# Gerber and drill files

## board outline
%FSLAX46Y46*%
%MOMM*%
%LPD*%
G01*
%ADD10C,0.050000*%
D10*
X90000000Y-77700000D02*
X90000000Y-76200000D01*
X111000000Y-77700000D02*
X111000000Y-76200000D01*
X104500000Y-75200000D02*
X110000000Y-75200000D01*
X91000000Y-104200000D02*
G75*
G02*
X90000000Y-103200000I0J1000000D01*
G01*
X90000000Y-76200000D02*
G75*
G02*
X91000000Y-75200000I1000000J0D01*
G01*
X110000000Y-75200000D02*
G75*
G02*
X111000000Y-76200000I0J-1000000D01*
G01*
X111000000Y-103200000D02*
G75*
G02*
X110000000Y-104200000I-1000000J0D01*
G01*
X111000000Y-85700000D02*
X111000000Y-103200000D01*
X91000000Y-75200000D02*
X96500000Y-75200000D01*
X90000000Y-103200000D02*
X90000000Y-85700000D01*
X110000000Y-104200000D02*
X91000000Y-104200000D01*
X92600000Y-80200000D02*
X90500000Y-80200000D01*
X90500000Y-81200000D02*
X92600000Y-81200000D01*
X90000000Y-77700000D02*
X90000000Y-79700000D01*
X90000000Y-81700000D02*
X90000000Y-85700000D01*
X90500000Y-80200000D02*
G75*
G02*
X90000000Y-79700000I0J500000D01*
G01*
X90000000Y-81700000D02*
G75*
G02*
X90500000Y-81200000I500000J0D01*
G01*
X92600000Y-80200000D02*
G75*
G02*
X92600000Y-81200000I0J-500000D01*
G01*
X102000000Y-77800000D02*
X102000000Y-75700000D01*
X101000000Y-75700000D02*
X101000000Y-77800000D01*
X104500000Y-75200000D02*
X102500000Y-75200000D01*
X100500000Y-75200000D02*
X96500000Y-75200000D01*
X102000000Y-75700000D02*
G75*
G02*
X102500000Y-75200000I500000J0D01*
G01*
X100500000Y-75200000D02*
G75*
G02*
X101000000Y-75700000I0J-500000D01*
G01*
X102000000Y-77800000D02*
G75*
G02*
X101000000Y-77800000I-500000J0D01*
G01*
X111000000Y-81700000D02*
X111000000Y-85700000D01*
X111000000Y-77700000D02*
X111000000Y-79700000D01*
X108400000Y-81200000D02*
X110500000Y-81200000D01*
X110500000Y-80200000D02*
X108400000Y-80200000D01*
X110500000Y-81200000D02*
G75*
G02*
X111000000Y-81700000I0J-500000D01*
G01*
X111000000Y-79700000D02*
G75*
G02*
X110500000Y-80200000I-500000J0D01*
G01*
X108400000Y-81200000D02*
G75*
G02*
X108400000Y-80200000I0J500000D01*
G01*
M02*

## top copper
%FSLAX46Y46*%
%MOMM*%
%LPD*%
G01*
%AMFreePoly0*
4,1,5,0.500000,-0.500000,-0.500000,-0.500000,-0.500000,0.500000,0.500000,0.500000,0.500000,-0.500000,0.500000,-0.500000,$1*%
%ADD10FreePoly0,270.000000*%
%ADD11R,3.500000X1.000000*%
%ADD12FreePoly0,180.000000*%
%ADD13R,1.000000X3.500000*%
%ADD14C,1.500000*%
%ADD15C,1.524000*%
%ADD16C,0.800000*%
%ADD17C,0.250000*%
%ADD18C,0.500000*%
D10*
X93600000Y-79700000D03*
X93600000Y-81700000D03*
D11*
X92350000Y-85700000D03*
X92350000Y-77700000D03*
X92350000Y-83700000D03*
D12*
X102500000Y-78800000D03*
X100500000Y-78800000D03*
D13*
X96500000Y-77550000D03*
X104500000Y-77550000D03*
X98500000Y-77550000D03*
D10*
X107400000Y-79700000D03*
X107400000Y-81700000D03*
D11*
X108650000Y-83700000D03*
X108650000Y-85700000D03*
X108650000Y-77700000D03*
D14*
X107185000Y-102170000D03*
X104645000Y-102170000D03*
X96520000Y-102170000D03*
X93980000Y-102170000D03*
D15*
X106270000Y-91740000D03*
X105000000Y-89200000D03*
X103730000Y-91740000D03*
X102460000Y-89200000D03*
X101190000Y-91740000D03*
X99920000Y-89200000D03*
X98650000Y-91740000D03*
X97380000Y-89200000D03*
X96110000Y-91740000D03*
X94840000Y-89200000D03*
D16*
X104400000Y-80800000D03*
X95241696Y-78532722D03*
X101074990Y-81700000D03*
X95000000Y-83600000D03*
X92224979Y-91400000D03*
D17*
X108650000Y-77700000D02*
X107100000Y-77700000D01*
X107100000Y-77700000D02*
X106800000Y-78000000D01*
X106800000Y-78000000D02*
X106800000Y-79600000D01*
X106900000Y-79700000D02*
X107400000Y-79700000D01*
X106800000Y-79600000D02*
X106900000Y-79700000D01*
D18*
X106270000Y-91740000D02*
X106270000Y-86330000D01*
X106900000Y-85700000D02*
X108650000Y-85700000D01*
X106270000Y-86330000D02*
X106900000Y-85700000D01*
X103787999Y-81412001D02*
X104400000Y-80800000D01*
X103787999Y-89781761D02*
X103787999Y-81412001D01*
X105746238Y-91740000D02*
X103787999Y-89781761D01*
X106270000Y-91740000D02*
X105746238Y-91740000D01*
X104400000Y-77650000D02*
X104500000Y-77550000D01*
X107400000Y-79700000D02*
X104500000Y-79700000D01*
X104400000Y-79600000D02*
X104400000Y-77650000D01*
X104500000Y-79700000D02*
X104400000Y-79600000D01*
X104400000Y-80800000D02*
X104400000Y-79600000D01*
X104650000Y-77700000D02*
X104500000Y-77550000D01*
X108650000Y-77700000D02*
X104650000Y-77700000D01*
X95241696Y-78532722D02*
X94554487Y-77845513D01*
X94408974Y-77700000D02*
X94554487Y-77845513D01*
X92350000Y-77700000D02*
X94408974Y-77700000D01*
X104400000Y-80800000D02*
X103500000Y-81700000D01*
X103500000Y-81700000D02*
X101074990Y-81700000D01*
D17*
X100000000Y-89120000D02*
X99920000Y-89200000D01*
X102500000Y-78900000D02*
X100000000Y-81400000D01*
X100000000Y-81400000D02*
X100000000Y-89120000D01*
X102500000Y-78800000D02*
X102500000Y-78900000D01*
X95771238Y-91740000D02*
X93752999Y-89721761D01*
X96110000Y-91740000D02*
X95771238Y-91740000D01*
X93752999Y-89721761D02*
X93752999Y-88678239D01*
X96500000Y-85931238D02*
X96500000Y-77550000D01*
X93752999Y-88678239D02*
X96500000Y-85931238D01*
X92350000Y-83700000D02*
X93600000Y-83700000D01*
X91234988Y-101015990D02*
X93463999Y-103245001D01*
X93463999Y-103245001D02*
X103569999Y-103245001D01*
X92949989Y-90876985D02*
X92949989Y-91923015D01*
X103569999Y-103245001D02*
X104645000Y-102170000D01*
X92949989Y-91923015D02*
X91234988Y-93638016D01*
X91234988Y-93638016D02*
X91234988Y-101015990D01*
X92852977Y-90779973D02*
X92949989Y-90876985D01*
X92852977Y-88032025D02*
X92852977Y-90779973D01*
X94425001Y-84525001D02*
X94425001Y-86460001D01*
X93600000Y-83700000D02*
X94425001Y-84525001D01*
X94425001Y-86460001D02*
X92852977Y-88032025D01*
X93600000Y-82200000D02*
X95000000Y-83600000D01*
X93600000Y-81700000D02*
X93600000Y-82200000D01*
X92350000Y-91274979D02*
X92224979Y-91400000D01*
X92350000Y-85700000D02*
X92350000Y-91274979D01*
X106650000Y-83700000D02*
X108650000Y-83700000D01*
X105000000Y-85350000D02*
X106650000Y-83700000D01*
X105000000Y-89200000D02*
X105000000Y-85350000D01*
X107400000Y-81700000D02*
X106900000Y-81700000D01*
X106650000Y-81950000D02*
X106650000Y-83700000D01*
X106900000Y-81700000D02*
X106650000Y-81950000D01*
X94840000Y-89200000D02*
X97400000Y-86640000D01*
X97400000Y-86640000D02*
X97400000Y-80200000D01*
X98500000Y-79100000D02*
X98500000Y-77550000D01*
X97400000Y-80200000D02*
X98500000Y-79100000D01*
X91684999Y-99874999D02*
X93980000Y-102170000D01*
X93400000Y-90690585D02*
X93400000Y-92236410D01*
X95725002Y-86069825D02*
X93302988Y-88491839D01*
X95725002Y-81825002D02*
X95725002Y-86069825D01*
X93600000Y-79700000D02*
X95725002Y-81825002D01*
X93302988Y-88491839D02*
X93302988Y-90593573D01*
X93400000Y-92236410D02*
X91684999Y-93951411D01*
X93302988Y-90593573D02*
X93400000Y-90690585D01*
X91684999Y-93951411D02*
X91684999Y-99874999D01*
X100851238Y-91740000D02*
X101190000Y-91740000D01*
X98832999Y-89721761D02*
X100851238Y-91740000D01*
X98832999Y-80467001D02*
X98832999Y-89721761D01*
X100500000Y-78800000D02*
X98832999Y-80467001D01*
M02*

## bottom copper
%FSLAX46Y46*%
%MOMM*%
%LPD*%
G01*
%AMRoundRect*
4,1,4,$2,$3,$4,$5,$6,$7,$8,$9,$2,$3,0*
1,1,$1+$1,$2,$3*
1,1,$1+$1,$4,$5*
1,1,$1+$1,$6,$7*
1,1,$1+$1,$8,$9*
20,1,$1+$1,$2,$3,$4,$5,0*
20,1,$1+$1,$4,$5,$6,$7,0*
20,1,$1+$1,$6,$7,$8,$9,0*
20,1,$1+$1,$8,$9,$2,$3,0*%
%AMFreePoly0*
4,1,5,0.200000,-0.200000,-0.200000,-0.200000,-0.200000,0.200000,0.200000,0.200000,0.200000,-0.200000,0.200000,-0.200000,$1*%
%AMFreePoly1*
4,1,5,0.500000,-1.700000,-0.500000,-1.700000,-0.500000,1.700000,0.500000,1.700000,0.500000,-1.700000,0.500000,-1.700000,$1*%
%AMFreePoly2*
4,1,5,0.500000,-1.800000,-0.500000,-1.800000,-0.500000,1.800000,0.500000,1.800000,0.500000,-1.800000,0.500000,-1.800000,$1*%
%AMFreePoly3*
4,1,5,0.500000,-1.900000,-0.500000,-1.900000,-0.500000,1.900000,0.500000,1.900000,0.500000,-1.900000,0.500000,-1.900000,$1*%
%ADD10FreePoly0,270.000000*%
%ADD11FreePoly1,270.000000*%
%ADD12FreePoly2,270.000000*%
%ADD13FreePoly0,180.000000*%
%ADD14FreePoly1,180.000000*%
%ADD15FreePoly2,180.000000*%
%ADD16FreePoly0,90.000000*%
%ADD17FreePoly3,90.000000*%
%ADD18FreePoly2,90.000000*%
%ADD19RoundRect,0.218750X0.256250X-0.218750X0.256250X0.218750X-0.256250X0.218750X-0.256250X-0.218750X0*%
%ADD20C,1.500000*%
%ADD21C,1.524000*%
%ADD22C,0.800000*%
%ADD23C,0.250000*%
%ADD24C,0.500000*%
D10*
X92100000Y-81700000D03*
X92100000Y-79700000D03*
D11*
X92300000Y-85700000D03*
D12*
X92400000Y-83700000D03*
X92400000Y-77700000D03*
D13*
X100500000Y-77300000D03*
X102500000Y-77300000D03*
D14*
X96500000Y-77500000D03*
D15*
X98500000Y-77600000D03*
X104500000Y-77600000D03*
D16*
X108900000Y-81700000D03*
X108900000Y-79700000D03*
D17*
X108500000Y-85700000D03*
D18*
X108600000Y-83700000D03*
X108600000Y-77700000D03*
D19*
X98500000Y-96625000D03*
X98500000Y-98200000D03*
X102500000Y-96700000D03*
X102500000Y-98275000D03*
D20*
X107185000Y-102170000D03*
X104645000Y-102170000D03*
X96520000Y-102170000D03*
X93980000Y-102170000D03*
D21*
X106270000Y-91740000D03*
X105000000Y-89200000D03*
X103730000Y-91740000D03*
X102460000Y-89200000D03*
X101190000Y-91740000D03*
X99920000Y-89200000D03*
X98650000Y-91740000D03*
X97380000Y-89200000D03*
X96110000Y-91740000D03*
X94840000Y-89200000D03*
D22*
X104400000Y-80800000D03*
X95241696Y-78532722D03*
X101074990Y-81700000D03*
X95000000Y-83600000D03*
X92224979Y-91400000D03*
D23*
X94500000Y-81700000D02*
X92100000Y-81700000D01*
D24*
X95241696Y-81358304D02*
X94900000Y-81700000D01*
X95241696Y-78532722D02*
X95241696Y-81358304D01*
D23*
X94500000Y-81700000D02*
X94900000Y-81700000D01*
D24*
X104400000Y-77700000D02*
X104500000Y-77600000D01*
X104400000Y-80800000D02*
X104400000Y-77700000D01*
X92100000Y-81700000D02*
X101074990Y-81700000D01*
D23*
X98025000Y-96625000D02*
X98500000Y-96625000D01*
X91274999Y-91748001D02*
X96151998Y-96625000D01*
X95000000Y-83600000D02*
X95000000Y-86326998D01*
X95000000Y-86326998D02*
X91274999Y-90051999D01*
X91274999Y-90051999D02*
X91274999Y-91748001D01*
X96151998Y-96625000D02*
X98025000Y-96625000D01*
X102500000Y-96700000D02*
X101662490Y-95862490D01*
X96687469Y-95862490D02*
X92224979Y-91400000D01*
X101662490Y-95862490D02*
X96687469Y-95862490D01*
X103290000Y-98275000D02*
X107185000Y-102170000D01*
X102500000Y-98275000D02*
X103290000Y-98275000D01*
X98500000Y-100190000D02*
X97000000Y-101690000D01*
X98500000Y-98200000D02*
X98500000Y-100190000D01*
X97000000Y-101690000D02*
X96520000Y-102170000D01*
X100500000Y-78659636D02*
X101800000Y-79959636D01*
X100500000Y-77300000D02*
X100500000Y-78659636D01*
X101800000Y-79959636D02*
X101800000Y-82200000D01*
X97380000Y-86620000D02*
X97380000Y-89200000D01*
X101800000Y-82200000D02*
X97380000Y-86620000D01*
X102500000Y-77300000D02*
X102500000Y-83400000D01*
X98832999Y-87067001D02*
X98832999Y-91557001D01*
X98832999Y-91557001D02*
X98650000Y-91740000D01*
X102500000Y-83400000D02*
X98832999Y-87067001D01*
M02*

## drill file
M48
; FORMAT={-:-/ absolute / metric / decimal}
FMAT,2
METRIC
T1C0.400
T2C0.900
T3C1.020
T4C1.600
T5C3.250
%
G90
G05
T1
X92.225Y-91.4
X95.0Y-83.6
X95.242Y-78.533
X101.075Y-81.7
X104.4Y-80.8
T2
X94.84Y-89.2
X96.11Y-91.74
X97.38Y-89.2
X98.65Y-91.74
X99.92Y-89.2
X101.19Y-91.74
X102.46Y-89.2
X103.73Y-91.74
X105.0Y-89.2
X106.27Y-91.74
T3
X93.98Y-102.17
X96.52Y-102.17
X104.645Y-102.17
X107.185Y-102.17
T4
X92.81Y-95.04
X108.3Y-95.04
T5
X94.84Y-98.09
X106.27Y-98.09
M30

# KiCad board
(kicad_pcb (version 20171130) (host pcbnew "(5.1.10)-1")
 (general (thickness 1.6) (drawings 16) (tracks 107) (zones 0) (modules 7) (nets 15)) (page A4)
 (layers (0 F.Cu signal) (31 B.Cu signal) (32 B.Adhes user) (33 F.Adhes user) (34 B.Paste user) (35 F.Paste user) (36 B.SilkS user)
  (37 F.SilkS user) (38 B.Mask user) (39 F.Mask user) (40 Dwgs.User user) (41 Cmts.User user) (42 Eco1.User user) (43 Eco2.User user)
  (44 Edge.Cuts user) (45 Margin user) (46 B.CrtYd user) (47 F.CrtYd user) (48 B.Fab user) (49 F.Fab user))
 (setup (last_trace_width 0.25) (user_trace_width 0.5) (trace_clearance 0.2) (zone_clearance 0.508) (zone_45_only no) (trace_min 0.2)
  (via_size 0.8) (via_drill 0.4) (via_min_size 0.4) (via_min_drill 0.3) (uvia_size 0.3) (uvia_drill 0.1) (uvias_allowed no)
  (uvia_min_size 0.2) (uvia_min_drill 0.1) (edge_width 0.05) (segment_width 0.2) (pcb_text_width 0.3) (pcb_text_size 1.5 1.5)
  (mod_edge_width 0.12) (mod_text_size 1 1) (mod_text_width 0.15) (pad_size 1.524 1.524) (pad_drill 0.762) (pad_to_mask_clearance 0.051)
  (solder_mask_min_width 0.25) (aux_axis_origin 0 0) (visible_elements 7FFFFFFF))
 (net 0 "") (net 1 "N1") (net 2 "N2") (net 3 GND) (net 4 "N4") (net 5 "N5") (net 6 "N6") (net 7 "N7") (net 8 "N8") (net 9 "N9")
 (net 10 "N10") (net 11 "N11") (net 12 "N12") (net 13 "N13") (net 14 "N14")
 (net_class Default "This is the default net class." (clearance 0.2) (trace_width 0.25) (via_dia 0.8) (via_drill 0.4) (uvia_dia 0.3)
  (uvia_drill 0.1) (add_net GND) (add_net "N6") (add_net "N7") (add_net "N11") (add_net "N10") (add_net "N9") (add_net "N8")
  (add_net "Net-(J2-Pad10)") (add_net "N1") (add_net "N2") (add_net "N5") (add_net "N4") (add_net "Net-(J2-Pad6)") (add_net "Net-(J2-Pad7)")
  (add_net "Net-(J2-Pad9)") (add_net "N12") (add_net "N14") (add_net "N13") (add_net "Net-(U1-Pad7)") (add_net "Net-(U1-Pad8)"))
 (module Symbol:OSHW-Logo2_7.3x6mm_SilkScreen (layer B.Cu) (at 100.2 83.6 180)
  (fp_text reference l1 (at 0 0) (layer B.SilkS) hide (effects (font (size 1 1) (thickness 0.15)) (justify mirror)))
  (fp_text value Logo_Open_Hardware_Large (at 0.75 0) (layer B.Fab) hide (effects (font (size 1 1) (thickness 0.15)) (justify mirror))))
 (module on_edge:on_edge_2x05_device (layer F.Cu) (at 90 81.7 270)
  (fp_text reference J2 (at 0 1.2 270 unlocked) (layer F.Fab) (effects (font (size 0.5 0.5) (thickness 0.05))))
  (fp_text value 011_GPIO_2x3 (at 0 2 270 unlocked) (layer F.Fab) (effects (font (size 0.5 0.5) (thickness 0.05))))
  (fp_line (start -1.5 -2.6) (end -1.5 -0.5) (layer Edge.Cuts) (width 0.05))
  (fp_line (start -0.5 -0.5) (end -0.5 -2.6) (layer Edge.Cuts) (width 0.05))
  (fp_line (start -4 0) (end -2 0) (layer Edge.Cuts) (width 0.05))
  (fp_line (start 0 0) (end 4 0) (layer Edge.Cuts) (width 0.05))
  (fp_arc (start -2 -0.5) (end -2 0) (angle -90) (layer Edge.Cuts) (width 0.05))
  (fp_arc (start 0 -0.5) (end -0.5 -0.5) (angle -90) (layer Edge.Cuts) (width 0.05))
  (fp_arc (start -1 -2.6) (end -0.5 -2.6) (angle -180) (layer Edge.Cuts) (width 0.05))
  (pad 2 smd custom (at -2 -3.6 270) (size 1 1) (layers F.Cu F.Mask) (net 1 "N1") (zone_connect 0)
   (options (clearance outline) (anchor rect)) (primitives))
  (pad 3 smd custom (at 0 -3.6 270) (size 1 1) (layers F.Cu F.Mask) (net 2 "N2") (zone_connect 0)
   (options (clearance outline) (anchor rect)) (primitives))
  (pad 8 smd custom (at 0 -2.1 270) (size 0.4 0.4) (layers B.Cu B.Mask) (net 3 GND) (zone_connect 0)
   (options (clearance outline) (anchor rect)) (primitives))
  (pad 7 smd custom (at -2 -2.1 270) (size 0.4 0.4) (layers B.Cu B.Mask) (zone_connect 0) (options (clearance outline) (anchor rect))
   (primitives))
  (pad 10 smd custom (at 4 -2.3 270) (size 1 3.4) (layers B.Cu B.Mask) (zone_connect 0) (options (clearance outline) (anchor rect))
   (primitives))
  (pad 9 smd custom (at 2 -2.4 270) (size 1 3.6) (layers B.Cu B.Mask) (zone_connect 0) (options (clearance outline) (anchor rect))
   (primitives))
  (pad 6 smd custom (at -4 -2.4 270) (size 1 3.6) (layers B.Cu B.Mask) (zone_connect 0) (options (clearance outline) (anchor rect))
   (primitives))
  (pad 5 smd rect (at 4 -2.35 90) (size 1 3.5) (layers F.Cu F.Mask) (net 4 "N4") (zone_connect 0))
  (pad 1 smd rect (at -4 -2.35 90) (size 1 3.5) (layers F.Cu F.Mask) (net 3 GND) (zone_connect 0))
  (pad 4 smd rect (at 2 -2.35 90) (size 1 3.5) (layers F.Cu F.Mask) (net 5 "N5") (zone_connect 0)))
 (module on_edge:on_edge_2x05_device (layer F.Cu) (at 100.5 75.2 180)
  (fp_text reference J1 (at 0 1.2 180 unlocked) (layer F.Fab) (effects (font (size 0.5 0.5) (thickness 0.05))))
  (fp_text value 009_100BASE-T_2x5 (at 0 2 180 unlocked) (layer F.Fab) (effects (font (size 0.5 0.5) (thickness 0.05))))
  (fp_line (start -1.5 -2.6) (end -1.5 -0.5) (layer Edge.Cuts) (width 0.05))
  (fp_line (start -0.5 -0.5) (end -0.5 -2.6) (layer Edge.Cuts) (width 0.05))
  (fp_line (start -4 0) (end -2 0) (layer Edge.Cuts) (width 0.05))
  (fp_line (start 0 0) (end 4 0) (layer Edge.Cuts) (width 0.05))
  (fp_arc (start -2 -0.5) (end -2 0) (angle -90) (layer Edge.Cuts) (width 0.05))
  (fp_arc (start 0 -0.5) (end -0.5 -0.5) (angle -90) (layer Edge.Cuts) (width 0.05))
  (fp_arc (start -1 -2.6) (end -0.5 -2.6) (angle -180) (layer Edge.Cuts) (width 0.05))
  (pad 2 smd custom (at -2 -3.6 180) (size 1 1) (layers F.Cu F.Mask) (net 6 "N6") (zone_connect 0)
   (options (clearance outline) (anchor rect)) (primitives))
  (pad 3 smd custom (at 0 -3.6 180) (size 1 1) (layers F.Cu F.Mask) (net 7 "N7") (zone_connect 0)
   (options (clearance outline) (anchor rect)) (primitives))
  (pad 8 smd custom (at 0 -2.1 180) (size 0.4 0.4) (layers B.Cu B.Mask) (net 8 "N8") (zone_connect 0)
   (options (clearance outline) (anchor rect)) (primitives))
  (pad 7 smd custom (at -2 -2.1 180) (size 0.4 0.4) (layers B.Cu B.Mask) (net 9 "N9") (zone_connect 0)
   (options (clearance outline) (anchor rect)) (primitives))
  (pad 10 smd custom (at 4 -2.3 180) (size 1 3.4) (layers B.Cu B.Mask) (zone_connect 0) (options (clearance outline) (anchor rect))
   (primitives))
  (pad 9 smd custom (at 2 -2.4 180) (size 1 3.6) (layers B.Cu B.Mask) (zone_connect 0) (options (clearance outline) (anchor rect))
   (primitives))
  (pad 6 smd custom (at -4 -2.4 180) (size 1 3.6) (layers B.Cu B.Mask) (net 3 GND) (zone_connect 0)
   (options (clearance outline) (anchor rect)) (primitives))
  (pad 5 smd rect (at 4 -2.35) (size 1 3.5) (layers F.Cu F.Mask) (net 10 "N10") (zone_connect 0))
  (pad 1 smd rect (at -4 -2.35) (size 1 3.5) (layers F.Cu F.Mask) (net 3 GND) (zone_connect 0))
  (pad 4 smd rect (at 2 -2.35) (size 1 3.5) (layers F.Cu F.Mask) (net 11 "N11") (zone_connect 0)))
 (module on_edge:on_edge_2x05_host (layer F.Cu) (at 111 81.7 270)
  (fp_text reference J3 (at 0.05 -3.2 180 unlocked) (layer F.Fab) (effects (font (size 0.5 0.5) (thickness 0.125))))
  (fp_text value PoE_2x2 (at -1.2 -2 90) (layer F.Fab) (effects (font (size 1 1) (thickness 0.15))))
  (fp_line (start 0 0) (end 4 0) (layer Edge.Cuts) (width 0.05))
  (fp_line (start -4 0) (end -2 0) (layer Edge.Cuts) (width 0.05))
  (fp_line (start -0.5 2.6) (end -0.5 0.5) (layer Edge.Cuts) (width 0.05))
  (fp_line (start -1.5 0.5) (end -1.5 2.6) (layer Edge.Cuts) (width 0.05))
  (fp_arc (start 0 0.5) (end 0 0) (angle -90) (layer Edge.Cuts) (width 0.05))
  (fp_arc (start -2 0.5) (end -1.5 0.5) (angle -90) (layer Edge.Cuts) (width 0.05))
  (fp_arc (start -1 2.6) (end -1.5 2.6) (angle -180) (layer Edge.Cuts) (width 0.05))
  (pad 2 smd custom (at -2 3.6 270) (size 1 1) (layers F.Cu F.Mask) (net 3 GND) (zone_connect 0) (options (clearance outline) (anchor rect))
   (primitives))
  (pad 3 smd custom (at 0 3.6 270) (size 1 1) (layers F.Cu F.Mask) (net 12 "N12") (zone_connect 0)
   (options (clearance outline) (anchor rect)) (primitives))
  (pad 8 smd custom (at 0 2.1 90) (size 0.4 0.4) (layers B.Cu B.Mask) (zone_connect 0) (options (clearance outline) (anchor rect))
   (primitives))
  (pad 7 smd custom (at -2 2.1 90) (size 0.4 0.4) (layers B.Cu B.Mask) (zone_connect 0) (options (clearance outline) (anchor rect))
   (primitives))
  (pad 4 smd rect (at 2 2.35 270) (size 1 3.5) (layers F.Cu F.Mask) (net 12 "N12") (zone_connect 0))
  (pad 10 smd custom (at 4 2.5 90) (size 1 3.8) (layers B.Cu B.Mask) (zone_connect 0) (options (clearance outline) (anchor rect))
   (primitives))
  (pad 9 smd custom (at 2 2.4 90) (size 1 3.6) (layers B.Cu B.Mask) (zone_connect 0) (options (clearance outline) (anchor rect))
   (primitives))
  (pad 6 smd custom (at -4 2.4 90) (size 1 3.6) (layers B.Cu B.Mask) (zone_connect 0) (options (clearance outline) (anchor rect))
   (primitives))
  (pad 5 smd rect (at 4 2.35 270) (size 1 3.5) (layers F.Cu F.Mask) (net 3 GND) (zone_connect 0))
  (pad 1 smd rect (at -4 2.35 270) (size 1 3.5) (layers F.Cu F.Mask) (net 3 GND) (zone_connect 0)))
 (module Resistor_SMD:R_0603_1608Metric (layer B.Cu) (at 98.5 97.4125 90)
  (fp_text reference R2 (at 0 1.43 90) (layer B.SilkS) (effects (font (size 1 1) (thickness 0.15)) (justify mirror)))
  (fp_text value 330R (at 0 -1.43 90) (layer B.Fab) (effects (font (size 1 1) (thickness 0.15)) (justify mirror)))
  (pad 2 smd roundrect (at 0.7875 0 90) (size 0.875 0.95) (layers B.Cu B.Paste B.Mask) (roundrect_rratio 0.25) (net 2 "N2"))
  (pad 1 smd roundrect (at -0.7875 0 90) (size 0.875 0.95) (layers B.Cu B.Paste B.Mask) (roundrect_rratio 0.25) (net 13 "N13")))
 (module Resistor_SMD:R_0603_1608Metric (layer B.Cu) (at 102.5 97.4875 90)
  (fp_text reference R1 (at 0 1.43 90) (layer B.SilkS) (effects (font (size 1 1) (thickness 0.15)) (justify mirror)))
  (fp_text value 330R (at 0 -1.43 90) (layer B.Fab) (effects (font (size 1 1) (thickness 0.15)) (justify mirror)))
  (pad 2 smd roundrect (at 0.7875 0 90) (size 0.875 0.95) (layers B.Cu B.Paste B.Mask) (roundrect_rratio 0.25) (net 4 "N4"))
  (pad 1 smd roundrect (at -0.7875 0 90) (size 0.875 0.95) (layers B.Cu B.Paste B.Mask) (roundrect_rratio 0.25) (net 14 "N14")))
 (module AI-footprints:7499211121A (layer F.Cu) (at 105 89.2 180)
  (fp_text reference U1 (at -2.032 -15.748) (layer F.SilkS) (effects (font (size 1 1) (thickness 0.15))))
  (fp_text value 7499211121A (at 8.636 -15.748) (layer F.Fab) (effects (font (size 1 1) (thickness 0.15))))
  (pad 14 thru_hole circle (at -2.185 -12.97 180) (size 1.5 1.5) (drill 1.02) (layers *.Cu *.Mask) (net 14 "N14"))
  (pad 13 thru_hole circle (at 0.355 -12.97 180) (size 1.5 1.5) (drill 1.02) (layers *.Cu *.Mask) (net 5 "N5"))
  (pad 12 thru_hole circle (at 8.48 -12.97 180) (size 1.5 1.5) (drill 1.02) (layers *.Cu *.Mask) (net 13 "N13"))
  (pad 11 thru_hole circle (at 11.02 -12.97 180) (size 1.5 1.5) (drill 1.02) (layers *.Cu *.Mask) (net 1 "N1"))
  (pad "" np_thru_hole circle (at 12.19 -5.84 180) (size 1.6 1.6) (drill 1.6) (layers *.Cu *.Mask))
  (pad "" np_thru_hole circle (at -3.3 -5.84 180) (size 1.6 1.6) (drill 1.6) (layers *.Cu *.Mask))
  (pad "" np_thru_hole circle (at 10.16 -8.89 180) (size 3.25 3.25) (drill 3.25) (layers *.Cu *.Mask))
  (pad "" np_thru_hole circle (at -1.27 -8.89 180) (size 3.25 3.25) (drill 3.25) (layers *.Cu *.Mask))
  (pad 10 thru_hole circle (at -1.27 -2.54 180) (size 1.524 1.524) (drill 0.9) (layers *.Cu *.Mask) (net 3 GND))
  (pad 9 thru_hole circle (at 0 0 180) (size 1.524 1.524) (drill 0.9) (layers *.Cu *.Mask) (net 12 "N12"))
  (pad 8 thru_hole circle (at 1.27 -2.54 180) (size 1.524 1.524) (drill 0.9) (layers *.Cu *.Mask))
  (pad 7 thru_hole circle (at 2.54 0 180) (size 1.524 1.524) (drill 0.9) (layers *.Cu *.Mask))
  (pad 6 thru_hole circle (at 3.81 -2.54 180) (size 1.524 1.524) (drill 0.9) (layers *.Cu *.Mask) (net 7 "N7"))
  (pad 5 thru_hole circle (at 5.08 0 180) (size 1.524 1.524) (drill 0.9) (layers *.Cu *.Mask) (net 6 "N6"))
  (pad 4 thru_hole circle (at 6.35 -2.54 180) (size 1.524 1.524) (drill 0.9) (layers *.Cu *.Mask) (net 9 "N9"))
  (pad 3 thru_hole circle (at 7.62 0 180) (size 1.524 1.524) (drill 0.9) (layers *.Cu *.Mask) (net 8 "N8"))
  (pad 2 thru_hole circle (at 8.89 -2.54 180) (size 1.524 1.524) (drill 0.9) (layers *.Cu *.Mask) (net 10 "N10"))
  (pad 1 thru_hole circle (at 10.16 0 180) (size 1.524 1.524) (drill 0.9) (layers *.Cu *.Mask) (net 11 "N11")))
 (gr_line (start 90 77.7) (end 90 76.2) (layer Edge.Cuts) (width 0.05))
 (gr_line (start 111 77.7) (end 111 76.2) (layer Edge.Cuts) (width 0.05))
 (gr_line (start 104.5 75.2) (end 110 75.2) (layer Edge.Cuts) (width 0.05))
 (gr_arc (start 91 103.2) (end 90 103.2) (angle -90) (layer Edge.Cuts) (width 0.05))
 (gr_arc (start 91 76.2) (end 91 75.2) (angle -90) (layer Edge.Cuts) (width 0.05))
 (gr_arc (start 110 76.2) (end 111 76.2) (angle -90) (layer Edge.Cuts) (width 0.05))
 (gr_arc (start 110 103.2) (end 110 104.2) (angle -90) (layer Edge.Cuts) (width 0.05))
 (gr_line (start 111 85.7) (end 111 103.2) (layer Edge.Cuts) (width 0.05))
 (gr_line (start 91 75.2) (end 96.5 75.2) (layer Edge.Cuts) (width 0.05))
 (gr_line (start 90 103.2) (end 90 85.7) (layer Edge.Cuts) (width 0.05))
 (gr_line (start 110 104.2) (end 91 104.2) (layer Edge.Cuts) (width 0.05))
 (segment (start 108.65 77.7) (end 107.1 77.7) (width 0.25) (layer F.Cu) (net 3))
 (segment (start 107.1 77.7) (end 106.8 78) (width 0.25) (layer F.Cu) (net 3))
 (segment (start 106.8 78) (end 106.8 79.6) (width 0.25) (layer F.Cu) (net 3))
 (segment (start 106.9 79.7) (end 107.4 79.7) (width 0.25) (layer F.Cu) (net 3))
 (segment (start 106.8 79.6) (end 106.9 79.7) (width 0.25) (layer F.Cu) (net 3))
 (via (at 104.4 80.8) (size 0.8) (drill 0.4) (layers F.Cu B.Cu) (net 3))
 (via (at 95.241696 78.532722) (size 0.8) (drill 0.4) (layers F.Cu B.Cu) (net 3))
 (segment (start 94.5 81.7) (end 92.1 81.7) (width 0.25) (layer B.Cu) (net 3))
 (segment (start 106.27 91.74) (end 106.27 86.33) (width 0.5) (layer F.Cu) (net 3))
 (segment (start 106.9 85.7) (end 108.65 85.7) (width 0.5) (layer F.Cu) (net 3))
 (segment (start 106.27 86.33) (end 106.9 85.7) (width 0.5) (layer F.Cu) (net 3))
 (segment (start 103.787999 81.412001) (end 104.4 80.8) (width 0.5) (layer F.Cu) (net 3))
 (segment (start 103.787999 89.781761) (end 103.787999 81.412001) (width 0.5) (layer F.Cu) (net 3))
 (segment (start 105.746238 91.74) (end 103.787999 89.781761) (width 0.5) (layer F.Cu) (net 3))
 (segment (start 106.27 91.74) (end 105.746238 91.74) (width 0.5) (layer F.Cu) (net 3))
 (segment (start 104.4 77.65) (end 104.5 77.55) (width 0.5) (layer F.Cu) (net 3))
 (segment (start 107.4 79.7) (end 104.5 79.7) (width 0.5) (layer F.Cu) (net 3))
 (segment (start 104.4 79.6) (end 104.4 77.65) (width 0.5) (layer F.Cu) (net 3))
 (segment (start 104.5 79.7) (end 104.4 79.6) (width 0.5) (layer F.Cu) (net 3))
 (segment (start 104.4 80.8) (end 104.4 79.6) (width 0.5) (layer F.Cu) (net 3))
 (segment (start 104.65 77.7) (end 104.5 77.55) (width 0.5) (layer F.Cu) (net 3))
 (segment (start 108.65 77.7) (end 104.65 77.7) (width 0.5) (layer F.Cu) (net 3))
 (segment (start 95.241696 78.532722) (end 94.554487 77.845513) (width 0.5) (layer F.Cu) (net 3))
 (segment (start 94.408974 77.7) (end 94.554487 77.845513) (width 0.5) (layer F.Cu) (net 3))
 (segment (start 92.35 77.7) (end 94.408974 77.7) (width 0.5) (layer F.Cu) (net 3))
 (segment (start 95.241696 81.358304) (end 94.9 81.7) (width 0.5) (layer B.Cu) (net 3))
 (segment (start 95.241696 78.532722) (end 95.241696 81.358304) (width 0.5) (layer B.Cu) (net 3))
 (segment (start 94.5 81.7) (end 94.9 81.7) (width 0.25) (layer B.Cu) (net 3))
 (segment (start 104.4 77.7) (end 104.5 77.6) (width 0.5) (layer B.Cu) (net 3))
 (segment (start 104.4 80.8) (end 104.4 77.7) (width 0.5) (layer B.Cu) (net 3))
 (via (at 101.07499 81.7) (size 0.8) (drill 0.4) (layers F.Cu B.Cu) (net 3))
 (segment (start 92.1 81.7) (end 101.07499 81.7) (width 0.5) (layer B.Cu) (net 3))
 (segment (start 104.4 80.8) (end 103.5 81.7) (width 0.5) (layer F.Cu) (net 3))
 (segment (start 103.5 81.7) (end 101.07499 81.7) (width 0.5) (layer F.Cu) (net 3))
 (segment (start 100 89.12) (end 99.92 89.2) (width 0.25) (layer F.Cu) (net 6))
 (segment (start 102.5 78.9) (end 100 81.4) (width 0.25) (layer F.Cu) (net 6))
 (segment (start 100 81.4) (end 100 89.12) (width 0.25) (layer F.Cu) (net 6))
 (segment (start 102.5 78.8) (end 102.5 78.9) (width 0.25) (layer F.Cu) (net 6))
 (segment (start 95.771238 91.74) (end 93.752999 89.721761) (width 0.25) (layer F.Cu) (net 10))
 (segment (start 96.11 91.74) (end 95.771238 91.74) (width 0.25) (layer F.Cu) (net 10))
 (segment (start 93.752999 89.721761) (end 93.752999 88.678239) (width 0.25) (layer F.Cu) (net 10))
 (segment (start 96.5 85.931238) (end 96.5 77.55) (width 0.25) (layer F.Cu) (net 10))
 (segment (start 93.752999 88.678239) (end 96.5 85.931238) (width 0.25) (layer F.Cu) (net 10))
 (segment (start 92.35 83.7) (end 93.6 83.7) (width 0.25) (layer F.Cu) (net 5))
 (segment (start 91.234988 101.01599) (end 93.463999 103.245001) (width 0.25) (layer F.Cu) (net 5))
 (segment (start 93.463999 103.245001) (end 103.569999 103.245001) (width 0.25) (layer F.Cu) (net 5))
 (segment (start 92.949989 90.876985) (end 92.949989 91.923015) (width 0.25) (layer F.Cu) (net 5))
 (segment (start 103.569999 103.245001) (end 104.645 102.17) (width 0.25) (layer F.Cu) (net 5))
 (segment (start 92.949989 91.923015) (end 91.234988 93.638016) (width 0.25) (layer F.Cu) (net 5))
 (segment (start 91.234988 93.638016) (end 91.234988 101.01599) (width 0.25) (layer F.Cu) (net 5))
 (segment (start 92.852977 90.779973) (end 92.949989 90.876985) (width 0.25) (layer F.Cu) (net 5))
 (segment (start 92.852977 88.032025) (end 92.852977 90.779973) (width 0.25) (layer F.Cu) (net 5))
 (segment (start 94.425001 84.525001) (end 94.425001 86.460001) (width 0.25) (layer F.Cu) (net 5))
 (segment (start 93.6 83.7) (end 94.425001 84.525001) (width 0.25) (layer F.Cu) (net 5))
 (segment (start 94.425001 86.460001) (end 92.852977 88.032025) (width 0.25) (layer F.Cu) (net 5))
 (segment (start 93.6 82.2) (end 95 83.6) (width 0.25) (layer F.Cu) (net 2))
 (via (at 95 83.6) (size 0.8) (drill 0.4) (layers F.Cu B.Cu) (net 2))
 (segment (start 93.6 81.7) (end 93.6 82.2) (width 0.25) (layer F.Cu) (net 2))
 (segment (start 98.025 96.625) (end 98.5 96.625) (width 0.25) (layer B.Cu) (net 2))
 (segment (start 91.274999 91.748001) (end 96.151998 96.625) (width 0.25) (layer B.Cu) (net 2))
 (segment (start 95 83.6) (end 95 86.326998) (width 0.25) (layer B.Cu) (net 2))
 (segment (start 95 86.326998) (end 91.274999 90.051999) (width 0.25) (layer B.Cu) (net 2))
 (segment (start 91.274999 90.051999) (end 91.274999 91.748001) (width 0.25) (layer B.Cu) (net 2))
 (segment (start 96.151998 96.625) (end 98.025 96.625) (width 0.25) (layer B.Cu) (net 2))
 (segment (start 92.35 91.274979) (end 92.224979 91.4) (width 0.25) (layer F.Cu) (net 4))
 (via (at 92.224979 91.4) (size 0.8) (drill 0.4) (layers F.Cu B.Cu) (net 4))
 (segment (start 102.5 96.7) (end 101.66249 95.86249) (width 0.25) (layer B.Cu) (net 4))
 (segment (start 96.687469 95.86249) (end 92.224979 91.4) (width 0.25) (layer B.Cu) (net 4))
 (segment (start 101.66249 95.86249) (end 96.687469 95.86249) (width 0.25) (layer B.Cu) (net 4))
 (segment (start 92.35 85.7) (end 92.35 91.274979) (width 0.25) (layer F.Cu) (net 4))
 (segment (start 106.65 83.7) (end 108.65 83.7) (width 0.25) (layer F.Cu) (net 12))
 (segment (start 105 85.35) (end 106.65 83.7) (width 0.25) (layer F.Cu) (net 12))
 (segment (start 105 89.2) (end 105 85.35) (width 0.25) (layer F.Cu) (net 12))
 (segment (start 107.4 81.7) (end 106.9 81.7) (width 0.25) (layer F.Cu) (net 12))
 (segment (start 106.65 81.95) (end 106.65 83.7) (width 0.25) (layer F.Cu) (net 12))
 (segment (start 106.9 81.7) (end 106.65 81.95) (width 0.25) (layer F.Cu) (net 12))
 (segment (start 103.29 98.275) (end 107.185 102.17) (width 0.25) (layer B.Cu) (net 14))
 (segment (start 102.5 98.275) (end 103.29 98.275) (width 0.25) (layer B.Cu) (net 14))
 (segment (start 98.5 100.19) (end 97 101.69) (width 0.25) (layer B.Cu) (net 13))
 (segment (start 98.5 98.2) (end 98.5 100.19) (width 0.25) (layer B.Cu) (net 13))
 (segment (start 97 101.69) (end 96.52 102.17) (width 0.25) (layer B.Cu) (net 13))
 (segment (start 94.84 89.2) (end 97.4 86.64) (width 0.25) (layer F.Cu) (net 11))
 (segment (start 97.4 86.64) (end 97.4 80.2) (width 0.25) (layer F.Cu) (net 11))
 (segment (start 98.5 79.1) (end 98.5 77.55) (width 0.25) (layer F.Cu) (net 11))
 (segment (start 97.4 80.2) (end 98.5 79.1) (width 0.25) (layer F.Cu) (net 11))
 (segment (start 91.684999 99.874999) (end 93.98 102.17) (width 0.25) (layer F.Cu) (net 1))
 (segment (start 93.4 90.690585) (end 93.4 92.23641) (width 0.25) (layer F.Cu) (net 1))
 (segment (start 95.725002 86.069825) (end 93.302988 88.491839) (width 0.25) (layer F.Cu) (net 1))
 (segment (start 95.725002 81.825002) (end 95.725002 86.069825) (width 0.25) (layer F.Cu) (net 1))
 (segment (start 93.6 79.7) (end 95.725002 81.825002) (width 0.25) (layer F.Cu) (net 1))
 (segment (start 93.302988 88.491839) (end 93.302988 90.593573) (width 0.25) (layer F.Cu) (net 1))
 (segment (start 93.4 92.23641) (end 91.684999 93.951411) (width 0.25) (layer F.Cu) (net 1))
 (segment (start 93.302988 90.593573) (end 93.4 90.690585) (width 0.25) (layer F.Cu) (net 1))
 (segment (start 91.684999 93.951411) (end 91.684999 99.874999) (width 0.25) (layer F.Cu) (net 1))
 (segment (start 100.851238 91.74) (end 101.19 91.74) (width 0.25) (layer F.Cu) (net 7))
 (segment (start 98.832999 89.721761) (end 100.851238 91.74) (width 0.25) (layer F.Cu) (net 7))
 (segment (start 98.832999 80.467001) (end 98.832999 89.721761) (width 0.25) (layer F.Cu) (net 7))
 (segment (start 100.5 78.8) (end 98.832999 80.467001) (width 0.25) (layer F.Cu) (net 7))
 (segment (start 100.5 78.659636) (end 101.8 79.959636) (width 0.25) (layer B.Cu) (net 8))
 (segment (start 100.5 77.3) (end 100.5 78.659636) (width 0.25) (layer B.Cu) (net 8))
 (segment (start 101.8 79.959636) (end 101.8 82.2) (width 0.25) (layer B.Cu) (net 8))
 (segment (start 97.38 86.62) (end 97.38 89.2) (width 0.25) (layer B.Cu) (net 8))
 (segment (start 101.8 82.2) (end 97.38 86.62) (width 0.25) (layer B.Cu) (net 8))
 (segment (start 102.5 77.3) (end 102.5 83.4) (width 0.25) (layer B.Cu) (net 9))
 (segment (start 98.832999 87.067001) (end 98.832999 91.557001) (width 0.25) (layer B.Cu) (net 9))
 (segment (start 98.832999 91.557001) (end 98.65 91.74) (width 0.25) (layer B.Cu) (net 9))
 (segment (start 102.5 83.4) (end 98.832999 87.067001) (width 0.25) (layer B.Cu) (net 9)))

